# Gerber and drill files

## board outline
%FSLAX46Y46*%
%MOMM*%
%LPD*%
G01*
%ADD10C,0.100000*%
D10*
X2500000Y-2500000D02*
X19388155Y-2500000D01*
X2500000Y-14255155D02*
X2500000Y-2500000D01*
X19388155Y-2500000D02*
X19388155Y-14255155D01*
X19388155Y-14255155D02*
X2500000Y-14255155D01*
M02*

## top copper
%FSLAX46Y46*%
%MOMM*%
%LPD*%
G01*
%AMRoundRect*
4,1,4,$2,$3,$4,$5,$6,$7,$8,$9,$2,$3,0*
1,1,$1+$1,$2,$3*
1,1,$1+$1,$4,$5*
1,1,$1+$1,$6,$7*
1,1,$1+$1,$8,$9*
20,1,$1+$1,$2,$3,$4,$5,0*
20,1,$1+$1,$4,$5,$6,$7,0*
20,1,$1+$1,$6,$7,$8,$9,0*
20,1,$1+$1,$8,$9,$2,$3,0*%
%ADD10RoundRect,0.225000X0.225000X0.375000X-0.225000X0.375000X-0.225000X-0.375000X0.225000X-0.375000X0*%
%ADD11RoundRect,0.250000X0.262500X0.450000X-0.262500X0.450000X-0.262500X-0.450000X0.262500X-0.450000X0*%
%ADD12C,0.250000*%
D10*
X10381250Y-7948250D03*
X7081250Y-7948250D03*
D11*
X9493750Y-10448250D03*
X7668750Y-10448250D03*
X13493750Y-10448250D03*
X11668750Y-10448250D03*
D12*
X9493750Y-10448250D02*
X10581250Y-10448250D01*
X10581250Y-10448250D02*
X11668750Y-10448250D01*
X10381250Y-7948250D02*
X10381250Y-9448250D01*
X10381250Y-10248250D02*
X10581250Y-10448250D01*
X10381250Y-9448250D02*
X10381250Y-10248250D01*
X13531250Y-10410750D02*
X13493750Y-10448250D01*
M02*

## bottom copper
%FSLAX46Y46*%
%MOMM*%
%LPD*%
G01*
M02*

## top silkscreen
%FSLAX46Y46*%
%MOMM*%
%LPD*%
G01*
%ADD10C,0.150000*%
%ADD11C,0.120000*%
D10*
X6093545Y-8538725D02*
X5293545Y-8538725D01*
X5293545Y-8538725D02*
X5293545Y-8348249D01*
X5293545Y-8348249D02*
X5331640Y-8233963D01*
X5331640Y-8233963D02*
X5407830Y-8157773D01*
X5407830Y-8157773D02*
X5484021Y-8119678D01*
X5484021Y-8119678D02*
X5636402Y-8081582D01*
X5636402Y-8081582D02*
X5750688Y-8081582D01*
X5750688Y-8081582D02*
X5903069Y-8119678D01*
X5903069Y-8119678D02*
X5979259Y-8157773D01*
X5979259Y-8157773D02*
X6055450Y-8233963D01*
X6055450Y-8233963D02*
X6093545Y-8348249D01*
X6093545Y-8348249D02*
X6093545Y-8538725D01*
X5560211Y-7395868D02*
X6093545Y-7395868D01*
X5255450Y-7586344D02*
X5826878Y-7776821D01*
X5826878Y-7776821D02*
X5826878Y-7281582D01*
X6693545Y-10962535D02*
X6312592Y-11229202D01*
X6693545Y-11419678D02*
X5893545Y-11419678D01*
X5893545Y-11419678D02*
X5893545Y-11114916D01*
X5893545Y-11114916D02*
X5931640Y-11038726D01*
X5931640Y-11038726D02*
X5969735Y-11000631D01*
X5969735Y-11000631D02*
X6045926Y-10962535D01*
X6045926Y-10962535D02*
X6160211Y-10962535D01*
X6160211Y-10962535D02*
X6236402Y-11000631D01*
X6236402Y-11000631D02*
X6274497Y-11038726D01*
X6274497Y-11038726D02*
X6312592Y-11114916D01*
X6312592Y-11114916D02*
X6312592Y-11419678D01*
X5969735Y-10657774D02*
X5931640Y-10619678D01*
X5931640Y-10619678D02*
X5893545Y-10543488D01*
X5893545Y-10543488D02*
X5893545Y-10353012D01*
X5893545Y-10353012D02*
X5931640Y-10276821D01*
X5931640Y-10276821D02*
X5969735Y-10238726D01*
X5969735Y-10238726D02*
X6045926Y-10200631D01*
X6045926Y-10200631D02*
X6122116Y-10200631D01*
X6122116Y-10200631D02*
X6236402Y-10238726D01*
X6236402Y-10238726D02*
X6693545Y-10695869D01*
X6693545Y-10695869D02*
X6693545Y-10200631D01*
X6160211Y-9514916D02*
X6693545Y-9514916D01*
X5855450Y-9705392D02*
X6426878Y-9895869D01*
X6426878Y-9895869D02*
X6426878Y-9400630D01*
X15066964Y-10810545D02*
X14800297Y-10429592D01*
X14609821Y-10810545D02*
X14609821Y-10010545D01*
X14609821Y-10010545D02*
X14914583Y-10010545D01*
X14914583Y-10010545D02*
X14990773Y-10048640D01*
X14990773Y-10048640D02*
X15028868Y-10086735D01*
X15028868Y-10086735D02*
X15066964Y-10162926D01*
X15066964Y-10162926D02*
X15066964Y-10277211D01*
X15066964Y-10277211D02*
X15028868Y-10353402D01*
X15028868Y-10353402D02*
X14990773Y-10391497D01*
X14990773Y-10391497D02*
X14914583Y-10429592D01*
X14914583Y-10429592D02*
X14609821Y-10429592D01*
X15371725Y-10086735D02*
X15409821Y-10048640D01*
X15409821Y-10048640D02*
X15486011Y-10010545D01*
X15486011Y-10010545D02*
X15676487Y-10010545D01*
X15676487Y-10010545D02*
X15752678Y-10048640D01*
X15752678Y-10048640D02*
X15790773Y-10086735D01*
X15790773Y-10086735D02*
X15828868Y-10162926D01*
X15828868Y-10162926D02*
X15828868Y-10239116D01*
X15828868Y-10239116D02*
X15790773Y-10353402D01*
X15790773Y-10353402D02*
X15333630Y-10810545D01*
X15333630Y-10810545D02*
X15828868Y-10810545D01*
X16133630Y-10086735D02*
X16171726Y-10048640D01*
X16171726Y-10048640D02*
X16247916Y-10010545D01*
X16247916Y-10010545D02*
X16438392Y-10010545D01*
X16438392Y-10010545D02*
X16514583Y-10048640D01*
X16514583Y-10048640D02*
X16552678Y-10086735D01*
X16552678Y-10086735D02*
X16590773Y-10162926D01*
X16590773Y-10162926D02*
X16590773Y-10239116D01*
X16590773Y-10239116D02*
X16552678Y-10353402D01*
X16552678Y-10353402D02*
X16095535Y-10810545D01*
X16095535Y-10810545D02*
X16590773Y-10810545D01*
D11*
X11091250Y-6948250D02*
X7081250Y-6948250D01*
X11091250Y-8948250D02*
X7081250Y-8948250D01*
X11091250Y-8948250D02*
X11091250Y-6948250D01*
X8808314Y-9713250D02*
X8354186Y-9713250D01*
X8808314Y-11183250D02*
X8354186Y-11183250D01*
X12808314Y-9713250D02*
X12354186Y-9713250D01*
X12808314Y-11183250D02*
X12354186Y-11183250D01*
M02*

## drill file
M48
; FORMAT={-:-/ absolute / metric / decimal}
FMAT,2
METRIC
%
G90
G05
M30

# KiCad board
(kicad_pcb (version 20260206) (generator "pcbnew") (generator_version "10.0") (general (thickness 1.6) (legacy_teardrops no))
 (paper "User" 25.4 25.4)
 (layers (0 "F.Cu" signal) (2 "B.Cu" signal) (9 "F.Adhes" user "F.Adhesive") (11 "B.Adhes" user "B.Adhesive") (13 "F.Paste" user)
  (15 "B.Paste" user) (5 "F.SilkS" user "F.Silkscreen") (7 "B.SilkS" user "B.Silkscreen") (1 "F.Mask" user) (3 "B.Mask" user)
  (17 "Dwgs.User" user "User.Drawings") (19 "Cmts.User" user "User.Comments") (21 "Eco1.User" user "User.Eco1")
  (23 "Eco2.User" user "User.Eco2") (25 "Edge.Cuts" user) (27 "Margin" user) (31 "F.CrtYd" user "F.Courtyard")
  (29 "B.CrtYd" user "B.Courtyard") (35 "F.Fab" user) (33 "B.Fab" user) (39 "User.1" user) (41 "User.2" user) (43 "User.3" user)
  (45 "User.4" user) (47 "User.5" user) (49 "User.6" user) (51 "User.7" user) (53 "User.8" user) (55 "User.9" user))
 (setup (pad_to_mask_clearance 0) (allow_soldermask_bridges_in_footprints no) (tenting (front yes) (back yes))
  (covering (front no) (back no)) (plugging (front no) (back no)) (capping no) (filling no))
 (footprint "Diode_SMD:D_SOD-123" (layer "F.Cu") (at 8.73125 7.94825 180)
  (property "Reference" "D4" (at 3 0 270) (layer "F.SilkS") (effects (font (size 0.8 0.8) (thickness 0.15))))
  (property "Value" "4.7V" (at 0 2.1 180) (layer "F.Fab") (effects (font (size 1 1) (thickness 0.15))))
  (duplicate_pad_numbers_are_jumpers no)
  (fp_line (start -2.36 1) (end 1.65 1) (stroke (width 0.12) (type solid)) (layer "F.SilkS"))
  (fp_line (start -2.36 -1) (end 1.65 -1) (stroke (width 0.12) (type solid)) (layer "F.SilkS"))
  (fp_line (start -2.36 -1) (end -2.36 1) (stroke (width 0.12) (type solid)) (layer "F.SilkS"))
  (pad "1" smd roundrect (at -1.65 0 180) (size 0.9 1.2) (layers "F.Cu" "F.Mask" "F.Paste") (roundrect_rratio 0.25) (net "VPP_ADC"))
  (pad "2" smd roundrect (at 1.65 0 180) (size 0.9 1.2) (layers "F.Cu" "F.Mask" "F.Paste") (roundrect_rratio 0.25) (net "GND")))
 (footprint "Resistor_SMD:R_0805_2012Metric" (layer "F.Cu") (at 8.58125 10.44825 180)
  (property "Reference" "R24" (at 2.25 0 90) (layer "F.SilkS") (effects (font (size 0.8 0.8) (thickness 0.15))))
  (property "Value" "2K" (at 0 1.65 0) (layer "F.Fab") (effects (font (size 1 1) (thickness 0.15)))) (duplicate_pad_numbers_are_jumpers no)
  (fp_line (start -0.227064 0.735) (end 0.227064 0.735) (stroke (width 0.12) (type solid)) (layer "F.SilkS"))
  (fp_line (start -0.227064 -0.735) (end 0.227064 -0.735) (stroke (width 0.12) (type solid)) (layer "F.SilkS"))
  (pad "1" smd roundrect (at -0.9125 0 180) (size 1.025 1.4) (layers "F.Cu" "F.Mask" "F.Paste") (roundrect_rratio 0.243902439)
   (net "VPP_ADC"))
  (pad "2" smd roundrect (at 0.9125 0 180) (size 1.025 1.4) (layers "F.Cu" "F.Mask" "F.Paste") (roundrect_rratio 0.243902439) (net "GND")))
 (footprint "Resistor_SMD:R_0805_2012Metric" (layer "F.Cu") (at 12.58125 10.44825 180)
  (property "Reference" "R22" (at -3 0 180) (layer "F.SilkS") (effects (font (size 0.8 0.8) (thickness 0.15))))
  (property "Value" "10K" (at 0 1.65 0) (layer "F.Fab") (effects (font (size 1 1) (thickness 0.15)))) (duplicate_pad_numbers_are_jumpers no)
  (fp_line (start -0.227064 0.735) (end 0.227064 0.735) (stroke (width 0.12) (type solid)) (layer "F.SilkS"))
  (fp_line (start -0.227064 -0.735) (end 0.227064 -0.735) (stroke (width 0.12) (type solid)) (layer "F.SilkS"))
  (pad "1" smd roundrect (at -0.9125 0 180) (size 1.025 1.4) (layers "F.Cu" "F.Mask" "F.Paste") (roundrect_rratio 0.243902439) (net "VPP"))
  (pad "2" smd roundrect (at 0.9125 0 180) (size 1.025 1.4) (layers "F.Cu" "F.Mask" "F.Paste") (roundrect_rratio 0.243902439)
   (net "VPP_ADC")))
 (gr_line (start 2.5 2.5) (end 19.388155 2.5) (stroke (width 0.1) (type default)) (layer "Edge.Cuts"))
 (gr_line (start 2.5 14.255155) (end 2.5 2.5) (stroke (width 0.1) (type default)) (layer "Edge.Cuts"))
 (gr_line (start 19.388155 2.5) (end 19.388155 14.255155) (stroke (width 0.1) (type default)) (layer "Edge.Cuts"))
 (gr_line (start 19.388155 14.255155) (end 2.5 14.255155) (stroke (width 0.1) (type default)) (layer "Edge.Cuts"))
 (segment (start 9.49375 10.44825) (end 10.58125 10.44825) (width 0.25) (layer "F.Cu") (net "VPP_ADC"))
 (segment (start 10.58125 10.44825) (end 11.66875 10.44825) (width 0.25) (layer "F.Cu") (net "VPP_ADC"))
 (segment (start 10.38125 7.94825) (end 10.38125 9.44825) (width 0.25) (layer "F.Cu") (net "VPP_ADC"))
 (segment (start 10.38125 10.24825) (end 10.58125 10.44825) (width 0.25) (layer "F.Cu") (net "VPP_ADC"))
 (segment (start 10.38125 9.44825) (end 10.38125 10.24825) (width 0.25) (layer "F.Cu") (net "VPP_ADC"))
 (segment (start 13.53125 10.41075) (end 13.49375 10.44825) (width 0.25) (layer "F.Cu") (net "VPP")))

